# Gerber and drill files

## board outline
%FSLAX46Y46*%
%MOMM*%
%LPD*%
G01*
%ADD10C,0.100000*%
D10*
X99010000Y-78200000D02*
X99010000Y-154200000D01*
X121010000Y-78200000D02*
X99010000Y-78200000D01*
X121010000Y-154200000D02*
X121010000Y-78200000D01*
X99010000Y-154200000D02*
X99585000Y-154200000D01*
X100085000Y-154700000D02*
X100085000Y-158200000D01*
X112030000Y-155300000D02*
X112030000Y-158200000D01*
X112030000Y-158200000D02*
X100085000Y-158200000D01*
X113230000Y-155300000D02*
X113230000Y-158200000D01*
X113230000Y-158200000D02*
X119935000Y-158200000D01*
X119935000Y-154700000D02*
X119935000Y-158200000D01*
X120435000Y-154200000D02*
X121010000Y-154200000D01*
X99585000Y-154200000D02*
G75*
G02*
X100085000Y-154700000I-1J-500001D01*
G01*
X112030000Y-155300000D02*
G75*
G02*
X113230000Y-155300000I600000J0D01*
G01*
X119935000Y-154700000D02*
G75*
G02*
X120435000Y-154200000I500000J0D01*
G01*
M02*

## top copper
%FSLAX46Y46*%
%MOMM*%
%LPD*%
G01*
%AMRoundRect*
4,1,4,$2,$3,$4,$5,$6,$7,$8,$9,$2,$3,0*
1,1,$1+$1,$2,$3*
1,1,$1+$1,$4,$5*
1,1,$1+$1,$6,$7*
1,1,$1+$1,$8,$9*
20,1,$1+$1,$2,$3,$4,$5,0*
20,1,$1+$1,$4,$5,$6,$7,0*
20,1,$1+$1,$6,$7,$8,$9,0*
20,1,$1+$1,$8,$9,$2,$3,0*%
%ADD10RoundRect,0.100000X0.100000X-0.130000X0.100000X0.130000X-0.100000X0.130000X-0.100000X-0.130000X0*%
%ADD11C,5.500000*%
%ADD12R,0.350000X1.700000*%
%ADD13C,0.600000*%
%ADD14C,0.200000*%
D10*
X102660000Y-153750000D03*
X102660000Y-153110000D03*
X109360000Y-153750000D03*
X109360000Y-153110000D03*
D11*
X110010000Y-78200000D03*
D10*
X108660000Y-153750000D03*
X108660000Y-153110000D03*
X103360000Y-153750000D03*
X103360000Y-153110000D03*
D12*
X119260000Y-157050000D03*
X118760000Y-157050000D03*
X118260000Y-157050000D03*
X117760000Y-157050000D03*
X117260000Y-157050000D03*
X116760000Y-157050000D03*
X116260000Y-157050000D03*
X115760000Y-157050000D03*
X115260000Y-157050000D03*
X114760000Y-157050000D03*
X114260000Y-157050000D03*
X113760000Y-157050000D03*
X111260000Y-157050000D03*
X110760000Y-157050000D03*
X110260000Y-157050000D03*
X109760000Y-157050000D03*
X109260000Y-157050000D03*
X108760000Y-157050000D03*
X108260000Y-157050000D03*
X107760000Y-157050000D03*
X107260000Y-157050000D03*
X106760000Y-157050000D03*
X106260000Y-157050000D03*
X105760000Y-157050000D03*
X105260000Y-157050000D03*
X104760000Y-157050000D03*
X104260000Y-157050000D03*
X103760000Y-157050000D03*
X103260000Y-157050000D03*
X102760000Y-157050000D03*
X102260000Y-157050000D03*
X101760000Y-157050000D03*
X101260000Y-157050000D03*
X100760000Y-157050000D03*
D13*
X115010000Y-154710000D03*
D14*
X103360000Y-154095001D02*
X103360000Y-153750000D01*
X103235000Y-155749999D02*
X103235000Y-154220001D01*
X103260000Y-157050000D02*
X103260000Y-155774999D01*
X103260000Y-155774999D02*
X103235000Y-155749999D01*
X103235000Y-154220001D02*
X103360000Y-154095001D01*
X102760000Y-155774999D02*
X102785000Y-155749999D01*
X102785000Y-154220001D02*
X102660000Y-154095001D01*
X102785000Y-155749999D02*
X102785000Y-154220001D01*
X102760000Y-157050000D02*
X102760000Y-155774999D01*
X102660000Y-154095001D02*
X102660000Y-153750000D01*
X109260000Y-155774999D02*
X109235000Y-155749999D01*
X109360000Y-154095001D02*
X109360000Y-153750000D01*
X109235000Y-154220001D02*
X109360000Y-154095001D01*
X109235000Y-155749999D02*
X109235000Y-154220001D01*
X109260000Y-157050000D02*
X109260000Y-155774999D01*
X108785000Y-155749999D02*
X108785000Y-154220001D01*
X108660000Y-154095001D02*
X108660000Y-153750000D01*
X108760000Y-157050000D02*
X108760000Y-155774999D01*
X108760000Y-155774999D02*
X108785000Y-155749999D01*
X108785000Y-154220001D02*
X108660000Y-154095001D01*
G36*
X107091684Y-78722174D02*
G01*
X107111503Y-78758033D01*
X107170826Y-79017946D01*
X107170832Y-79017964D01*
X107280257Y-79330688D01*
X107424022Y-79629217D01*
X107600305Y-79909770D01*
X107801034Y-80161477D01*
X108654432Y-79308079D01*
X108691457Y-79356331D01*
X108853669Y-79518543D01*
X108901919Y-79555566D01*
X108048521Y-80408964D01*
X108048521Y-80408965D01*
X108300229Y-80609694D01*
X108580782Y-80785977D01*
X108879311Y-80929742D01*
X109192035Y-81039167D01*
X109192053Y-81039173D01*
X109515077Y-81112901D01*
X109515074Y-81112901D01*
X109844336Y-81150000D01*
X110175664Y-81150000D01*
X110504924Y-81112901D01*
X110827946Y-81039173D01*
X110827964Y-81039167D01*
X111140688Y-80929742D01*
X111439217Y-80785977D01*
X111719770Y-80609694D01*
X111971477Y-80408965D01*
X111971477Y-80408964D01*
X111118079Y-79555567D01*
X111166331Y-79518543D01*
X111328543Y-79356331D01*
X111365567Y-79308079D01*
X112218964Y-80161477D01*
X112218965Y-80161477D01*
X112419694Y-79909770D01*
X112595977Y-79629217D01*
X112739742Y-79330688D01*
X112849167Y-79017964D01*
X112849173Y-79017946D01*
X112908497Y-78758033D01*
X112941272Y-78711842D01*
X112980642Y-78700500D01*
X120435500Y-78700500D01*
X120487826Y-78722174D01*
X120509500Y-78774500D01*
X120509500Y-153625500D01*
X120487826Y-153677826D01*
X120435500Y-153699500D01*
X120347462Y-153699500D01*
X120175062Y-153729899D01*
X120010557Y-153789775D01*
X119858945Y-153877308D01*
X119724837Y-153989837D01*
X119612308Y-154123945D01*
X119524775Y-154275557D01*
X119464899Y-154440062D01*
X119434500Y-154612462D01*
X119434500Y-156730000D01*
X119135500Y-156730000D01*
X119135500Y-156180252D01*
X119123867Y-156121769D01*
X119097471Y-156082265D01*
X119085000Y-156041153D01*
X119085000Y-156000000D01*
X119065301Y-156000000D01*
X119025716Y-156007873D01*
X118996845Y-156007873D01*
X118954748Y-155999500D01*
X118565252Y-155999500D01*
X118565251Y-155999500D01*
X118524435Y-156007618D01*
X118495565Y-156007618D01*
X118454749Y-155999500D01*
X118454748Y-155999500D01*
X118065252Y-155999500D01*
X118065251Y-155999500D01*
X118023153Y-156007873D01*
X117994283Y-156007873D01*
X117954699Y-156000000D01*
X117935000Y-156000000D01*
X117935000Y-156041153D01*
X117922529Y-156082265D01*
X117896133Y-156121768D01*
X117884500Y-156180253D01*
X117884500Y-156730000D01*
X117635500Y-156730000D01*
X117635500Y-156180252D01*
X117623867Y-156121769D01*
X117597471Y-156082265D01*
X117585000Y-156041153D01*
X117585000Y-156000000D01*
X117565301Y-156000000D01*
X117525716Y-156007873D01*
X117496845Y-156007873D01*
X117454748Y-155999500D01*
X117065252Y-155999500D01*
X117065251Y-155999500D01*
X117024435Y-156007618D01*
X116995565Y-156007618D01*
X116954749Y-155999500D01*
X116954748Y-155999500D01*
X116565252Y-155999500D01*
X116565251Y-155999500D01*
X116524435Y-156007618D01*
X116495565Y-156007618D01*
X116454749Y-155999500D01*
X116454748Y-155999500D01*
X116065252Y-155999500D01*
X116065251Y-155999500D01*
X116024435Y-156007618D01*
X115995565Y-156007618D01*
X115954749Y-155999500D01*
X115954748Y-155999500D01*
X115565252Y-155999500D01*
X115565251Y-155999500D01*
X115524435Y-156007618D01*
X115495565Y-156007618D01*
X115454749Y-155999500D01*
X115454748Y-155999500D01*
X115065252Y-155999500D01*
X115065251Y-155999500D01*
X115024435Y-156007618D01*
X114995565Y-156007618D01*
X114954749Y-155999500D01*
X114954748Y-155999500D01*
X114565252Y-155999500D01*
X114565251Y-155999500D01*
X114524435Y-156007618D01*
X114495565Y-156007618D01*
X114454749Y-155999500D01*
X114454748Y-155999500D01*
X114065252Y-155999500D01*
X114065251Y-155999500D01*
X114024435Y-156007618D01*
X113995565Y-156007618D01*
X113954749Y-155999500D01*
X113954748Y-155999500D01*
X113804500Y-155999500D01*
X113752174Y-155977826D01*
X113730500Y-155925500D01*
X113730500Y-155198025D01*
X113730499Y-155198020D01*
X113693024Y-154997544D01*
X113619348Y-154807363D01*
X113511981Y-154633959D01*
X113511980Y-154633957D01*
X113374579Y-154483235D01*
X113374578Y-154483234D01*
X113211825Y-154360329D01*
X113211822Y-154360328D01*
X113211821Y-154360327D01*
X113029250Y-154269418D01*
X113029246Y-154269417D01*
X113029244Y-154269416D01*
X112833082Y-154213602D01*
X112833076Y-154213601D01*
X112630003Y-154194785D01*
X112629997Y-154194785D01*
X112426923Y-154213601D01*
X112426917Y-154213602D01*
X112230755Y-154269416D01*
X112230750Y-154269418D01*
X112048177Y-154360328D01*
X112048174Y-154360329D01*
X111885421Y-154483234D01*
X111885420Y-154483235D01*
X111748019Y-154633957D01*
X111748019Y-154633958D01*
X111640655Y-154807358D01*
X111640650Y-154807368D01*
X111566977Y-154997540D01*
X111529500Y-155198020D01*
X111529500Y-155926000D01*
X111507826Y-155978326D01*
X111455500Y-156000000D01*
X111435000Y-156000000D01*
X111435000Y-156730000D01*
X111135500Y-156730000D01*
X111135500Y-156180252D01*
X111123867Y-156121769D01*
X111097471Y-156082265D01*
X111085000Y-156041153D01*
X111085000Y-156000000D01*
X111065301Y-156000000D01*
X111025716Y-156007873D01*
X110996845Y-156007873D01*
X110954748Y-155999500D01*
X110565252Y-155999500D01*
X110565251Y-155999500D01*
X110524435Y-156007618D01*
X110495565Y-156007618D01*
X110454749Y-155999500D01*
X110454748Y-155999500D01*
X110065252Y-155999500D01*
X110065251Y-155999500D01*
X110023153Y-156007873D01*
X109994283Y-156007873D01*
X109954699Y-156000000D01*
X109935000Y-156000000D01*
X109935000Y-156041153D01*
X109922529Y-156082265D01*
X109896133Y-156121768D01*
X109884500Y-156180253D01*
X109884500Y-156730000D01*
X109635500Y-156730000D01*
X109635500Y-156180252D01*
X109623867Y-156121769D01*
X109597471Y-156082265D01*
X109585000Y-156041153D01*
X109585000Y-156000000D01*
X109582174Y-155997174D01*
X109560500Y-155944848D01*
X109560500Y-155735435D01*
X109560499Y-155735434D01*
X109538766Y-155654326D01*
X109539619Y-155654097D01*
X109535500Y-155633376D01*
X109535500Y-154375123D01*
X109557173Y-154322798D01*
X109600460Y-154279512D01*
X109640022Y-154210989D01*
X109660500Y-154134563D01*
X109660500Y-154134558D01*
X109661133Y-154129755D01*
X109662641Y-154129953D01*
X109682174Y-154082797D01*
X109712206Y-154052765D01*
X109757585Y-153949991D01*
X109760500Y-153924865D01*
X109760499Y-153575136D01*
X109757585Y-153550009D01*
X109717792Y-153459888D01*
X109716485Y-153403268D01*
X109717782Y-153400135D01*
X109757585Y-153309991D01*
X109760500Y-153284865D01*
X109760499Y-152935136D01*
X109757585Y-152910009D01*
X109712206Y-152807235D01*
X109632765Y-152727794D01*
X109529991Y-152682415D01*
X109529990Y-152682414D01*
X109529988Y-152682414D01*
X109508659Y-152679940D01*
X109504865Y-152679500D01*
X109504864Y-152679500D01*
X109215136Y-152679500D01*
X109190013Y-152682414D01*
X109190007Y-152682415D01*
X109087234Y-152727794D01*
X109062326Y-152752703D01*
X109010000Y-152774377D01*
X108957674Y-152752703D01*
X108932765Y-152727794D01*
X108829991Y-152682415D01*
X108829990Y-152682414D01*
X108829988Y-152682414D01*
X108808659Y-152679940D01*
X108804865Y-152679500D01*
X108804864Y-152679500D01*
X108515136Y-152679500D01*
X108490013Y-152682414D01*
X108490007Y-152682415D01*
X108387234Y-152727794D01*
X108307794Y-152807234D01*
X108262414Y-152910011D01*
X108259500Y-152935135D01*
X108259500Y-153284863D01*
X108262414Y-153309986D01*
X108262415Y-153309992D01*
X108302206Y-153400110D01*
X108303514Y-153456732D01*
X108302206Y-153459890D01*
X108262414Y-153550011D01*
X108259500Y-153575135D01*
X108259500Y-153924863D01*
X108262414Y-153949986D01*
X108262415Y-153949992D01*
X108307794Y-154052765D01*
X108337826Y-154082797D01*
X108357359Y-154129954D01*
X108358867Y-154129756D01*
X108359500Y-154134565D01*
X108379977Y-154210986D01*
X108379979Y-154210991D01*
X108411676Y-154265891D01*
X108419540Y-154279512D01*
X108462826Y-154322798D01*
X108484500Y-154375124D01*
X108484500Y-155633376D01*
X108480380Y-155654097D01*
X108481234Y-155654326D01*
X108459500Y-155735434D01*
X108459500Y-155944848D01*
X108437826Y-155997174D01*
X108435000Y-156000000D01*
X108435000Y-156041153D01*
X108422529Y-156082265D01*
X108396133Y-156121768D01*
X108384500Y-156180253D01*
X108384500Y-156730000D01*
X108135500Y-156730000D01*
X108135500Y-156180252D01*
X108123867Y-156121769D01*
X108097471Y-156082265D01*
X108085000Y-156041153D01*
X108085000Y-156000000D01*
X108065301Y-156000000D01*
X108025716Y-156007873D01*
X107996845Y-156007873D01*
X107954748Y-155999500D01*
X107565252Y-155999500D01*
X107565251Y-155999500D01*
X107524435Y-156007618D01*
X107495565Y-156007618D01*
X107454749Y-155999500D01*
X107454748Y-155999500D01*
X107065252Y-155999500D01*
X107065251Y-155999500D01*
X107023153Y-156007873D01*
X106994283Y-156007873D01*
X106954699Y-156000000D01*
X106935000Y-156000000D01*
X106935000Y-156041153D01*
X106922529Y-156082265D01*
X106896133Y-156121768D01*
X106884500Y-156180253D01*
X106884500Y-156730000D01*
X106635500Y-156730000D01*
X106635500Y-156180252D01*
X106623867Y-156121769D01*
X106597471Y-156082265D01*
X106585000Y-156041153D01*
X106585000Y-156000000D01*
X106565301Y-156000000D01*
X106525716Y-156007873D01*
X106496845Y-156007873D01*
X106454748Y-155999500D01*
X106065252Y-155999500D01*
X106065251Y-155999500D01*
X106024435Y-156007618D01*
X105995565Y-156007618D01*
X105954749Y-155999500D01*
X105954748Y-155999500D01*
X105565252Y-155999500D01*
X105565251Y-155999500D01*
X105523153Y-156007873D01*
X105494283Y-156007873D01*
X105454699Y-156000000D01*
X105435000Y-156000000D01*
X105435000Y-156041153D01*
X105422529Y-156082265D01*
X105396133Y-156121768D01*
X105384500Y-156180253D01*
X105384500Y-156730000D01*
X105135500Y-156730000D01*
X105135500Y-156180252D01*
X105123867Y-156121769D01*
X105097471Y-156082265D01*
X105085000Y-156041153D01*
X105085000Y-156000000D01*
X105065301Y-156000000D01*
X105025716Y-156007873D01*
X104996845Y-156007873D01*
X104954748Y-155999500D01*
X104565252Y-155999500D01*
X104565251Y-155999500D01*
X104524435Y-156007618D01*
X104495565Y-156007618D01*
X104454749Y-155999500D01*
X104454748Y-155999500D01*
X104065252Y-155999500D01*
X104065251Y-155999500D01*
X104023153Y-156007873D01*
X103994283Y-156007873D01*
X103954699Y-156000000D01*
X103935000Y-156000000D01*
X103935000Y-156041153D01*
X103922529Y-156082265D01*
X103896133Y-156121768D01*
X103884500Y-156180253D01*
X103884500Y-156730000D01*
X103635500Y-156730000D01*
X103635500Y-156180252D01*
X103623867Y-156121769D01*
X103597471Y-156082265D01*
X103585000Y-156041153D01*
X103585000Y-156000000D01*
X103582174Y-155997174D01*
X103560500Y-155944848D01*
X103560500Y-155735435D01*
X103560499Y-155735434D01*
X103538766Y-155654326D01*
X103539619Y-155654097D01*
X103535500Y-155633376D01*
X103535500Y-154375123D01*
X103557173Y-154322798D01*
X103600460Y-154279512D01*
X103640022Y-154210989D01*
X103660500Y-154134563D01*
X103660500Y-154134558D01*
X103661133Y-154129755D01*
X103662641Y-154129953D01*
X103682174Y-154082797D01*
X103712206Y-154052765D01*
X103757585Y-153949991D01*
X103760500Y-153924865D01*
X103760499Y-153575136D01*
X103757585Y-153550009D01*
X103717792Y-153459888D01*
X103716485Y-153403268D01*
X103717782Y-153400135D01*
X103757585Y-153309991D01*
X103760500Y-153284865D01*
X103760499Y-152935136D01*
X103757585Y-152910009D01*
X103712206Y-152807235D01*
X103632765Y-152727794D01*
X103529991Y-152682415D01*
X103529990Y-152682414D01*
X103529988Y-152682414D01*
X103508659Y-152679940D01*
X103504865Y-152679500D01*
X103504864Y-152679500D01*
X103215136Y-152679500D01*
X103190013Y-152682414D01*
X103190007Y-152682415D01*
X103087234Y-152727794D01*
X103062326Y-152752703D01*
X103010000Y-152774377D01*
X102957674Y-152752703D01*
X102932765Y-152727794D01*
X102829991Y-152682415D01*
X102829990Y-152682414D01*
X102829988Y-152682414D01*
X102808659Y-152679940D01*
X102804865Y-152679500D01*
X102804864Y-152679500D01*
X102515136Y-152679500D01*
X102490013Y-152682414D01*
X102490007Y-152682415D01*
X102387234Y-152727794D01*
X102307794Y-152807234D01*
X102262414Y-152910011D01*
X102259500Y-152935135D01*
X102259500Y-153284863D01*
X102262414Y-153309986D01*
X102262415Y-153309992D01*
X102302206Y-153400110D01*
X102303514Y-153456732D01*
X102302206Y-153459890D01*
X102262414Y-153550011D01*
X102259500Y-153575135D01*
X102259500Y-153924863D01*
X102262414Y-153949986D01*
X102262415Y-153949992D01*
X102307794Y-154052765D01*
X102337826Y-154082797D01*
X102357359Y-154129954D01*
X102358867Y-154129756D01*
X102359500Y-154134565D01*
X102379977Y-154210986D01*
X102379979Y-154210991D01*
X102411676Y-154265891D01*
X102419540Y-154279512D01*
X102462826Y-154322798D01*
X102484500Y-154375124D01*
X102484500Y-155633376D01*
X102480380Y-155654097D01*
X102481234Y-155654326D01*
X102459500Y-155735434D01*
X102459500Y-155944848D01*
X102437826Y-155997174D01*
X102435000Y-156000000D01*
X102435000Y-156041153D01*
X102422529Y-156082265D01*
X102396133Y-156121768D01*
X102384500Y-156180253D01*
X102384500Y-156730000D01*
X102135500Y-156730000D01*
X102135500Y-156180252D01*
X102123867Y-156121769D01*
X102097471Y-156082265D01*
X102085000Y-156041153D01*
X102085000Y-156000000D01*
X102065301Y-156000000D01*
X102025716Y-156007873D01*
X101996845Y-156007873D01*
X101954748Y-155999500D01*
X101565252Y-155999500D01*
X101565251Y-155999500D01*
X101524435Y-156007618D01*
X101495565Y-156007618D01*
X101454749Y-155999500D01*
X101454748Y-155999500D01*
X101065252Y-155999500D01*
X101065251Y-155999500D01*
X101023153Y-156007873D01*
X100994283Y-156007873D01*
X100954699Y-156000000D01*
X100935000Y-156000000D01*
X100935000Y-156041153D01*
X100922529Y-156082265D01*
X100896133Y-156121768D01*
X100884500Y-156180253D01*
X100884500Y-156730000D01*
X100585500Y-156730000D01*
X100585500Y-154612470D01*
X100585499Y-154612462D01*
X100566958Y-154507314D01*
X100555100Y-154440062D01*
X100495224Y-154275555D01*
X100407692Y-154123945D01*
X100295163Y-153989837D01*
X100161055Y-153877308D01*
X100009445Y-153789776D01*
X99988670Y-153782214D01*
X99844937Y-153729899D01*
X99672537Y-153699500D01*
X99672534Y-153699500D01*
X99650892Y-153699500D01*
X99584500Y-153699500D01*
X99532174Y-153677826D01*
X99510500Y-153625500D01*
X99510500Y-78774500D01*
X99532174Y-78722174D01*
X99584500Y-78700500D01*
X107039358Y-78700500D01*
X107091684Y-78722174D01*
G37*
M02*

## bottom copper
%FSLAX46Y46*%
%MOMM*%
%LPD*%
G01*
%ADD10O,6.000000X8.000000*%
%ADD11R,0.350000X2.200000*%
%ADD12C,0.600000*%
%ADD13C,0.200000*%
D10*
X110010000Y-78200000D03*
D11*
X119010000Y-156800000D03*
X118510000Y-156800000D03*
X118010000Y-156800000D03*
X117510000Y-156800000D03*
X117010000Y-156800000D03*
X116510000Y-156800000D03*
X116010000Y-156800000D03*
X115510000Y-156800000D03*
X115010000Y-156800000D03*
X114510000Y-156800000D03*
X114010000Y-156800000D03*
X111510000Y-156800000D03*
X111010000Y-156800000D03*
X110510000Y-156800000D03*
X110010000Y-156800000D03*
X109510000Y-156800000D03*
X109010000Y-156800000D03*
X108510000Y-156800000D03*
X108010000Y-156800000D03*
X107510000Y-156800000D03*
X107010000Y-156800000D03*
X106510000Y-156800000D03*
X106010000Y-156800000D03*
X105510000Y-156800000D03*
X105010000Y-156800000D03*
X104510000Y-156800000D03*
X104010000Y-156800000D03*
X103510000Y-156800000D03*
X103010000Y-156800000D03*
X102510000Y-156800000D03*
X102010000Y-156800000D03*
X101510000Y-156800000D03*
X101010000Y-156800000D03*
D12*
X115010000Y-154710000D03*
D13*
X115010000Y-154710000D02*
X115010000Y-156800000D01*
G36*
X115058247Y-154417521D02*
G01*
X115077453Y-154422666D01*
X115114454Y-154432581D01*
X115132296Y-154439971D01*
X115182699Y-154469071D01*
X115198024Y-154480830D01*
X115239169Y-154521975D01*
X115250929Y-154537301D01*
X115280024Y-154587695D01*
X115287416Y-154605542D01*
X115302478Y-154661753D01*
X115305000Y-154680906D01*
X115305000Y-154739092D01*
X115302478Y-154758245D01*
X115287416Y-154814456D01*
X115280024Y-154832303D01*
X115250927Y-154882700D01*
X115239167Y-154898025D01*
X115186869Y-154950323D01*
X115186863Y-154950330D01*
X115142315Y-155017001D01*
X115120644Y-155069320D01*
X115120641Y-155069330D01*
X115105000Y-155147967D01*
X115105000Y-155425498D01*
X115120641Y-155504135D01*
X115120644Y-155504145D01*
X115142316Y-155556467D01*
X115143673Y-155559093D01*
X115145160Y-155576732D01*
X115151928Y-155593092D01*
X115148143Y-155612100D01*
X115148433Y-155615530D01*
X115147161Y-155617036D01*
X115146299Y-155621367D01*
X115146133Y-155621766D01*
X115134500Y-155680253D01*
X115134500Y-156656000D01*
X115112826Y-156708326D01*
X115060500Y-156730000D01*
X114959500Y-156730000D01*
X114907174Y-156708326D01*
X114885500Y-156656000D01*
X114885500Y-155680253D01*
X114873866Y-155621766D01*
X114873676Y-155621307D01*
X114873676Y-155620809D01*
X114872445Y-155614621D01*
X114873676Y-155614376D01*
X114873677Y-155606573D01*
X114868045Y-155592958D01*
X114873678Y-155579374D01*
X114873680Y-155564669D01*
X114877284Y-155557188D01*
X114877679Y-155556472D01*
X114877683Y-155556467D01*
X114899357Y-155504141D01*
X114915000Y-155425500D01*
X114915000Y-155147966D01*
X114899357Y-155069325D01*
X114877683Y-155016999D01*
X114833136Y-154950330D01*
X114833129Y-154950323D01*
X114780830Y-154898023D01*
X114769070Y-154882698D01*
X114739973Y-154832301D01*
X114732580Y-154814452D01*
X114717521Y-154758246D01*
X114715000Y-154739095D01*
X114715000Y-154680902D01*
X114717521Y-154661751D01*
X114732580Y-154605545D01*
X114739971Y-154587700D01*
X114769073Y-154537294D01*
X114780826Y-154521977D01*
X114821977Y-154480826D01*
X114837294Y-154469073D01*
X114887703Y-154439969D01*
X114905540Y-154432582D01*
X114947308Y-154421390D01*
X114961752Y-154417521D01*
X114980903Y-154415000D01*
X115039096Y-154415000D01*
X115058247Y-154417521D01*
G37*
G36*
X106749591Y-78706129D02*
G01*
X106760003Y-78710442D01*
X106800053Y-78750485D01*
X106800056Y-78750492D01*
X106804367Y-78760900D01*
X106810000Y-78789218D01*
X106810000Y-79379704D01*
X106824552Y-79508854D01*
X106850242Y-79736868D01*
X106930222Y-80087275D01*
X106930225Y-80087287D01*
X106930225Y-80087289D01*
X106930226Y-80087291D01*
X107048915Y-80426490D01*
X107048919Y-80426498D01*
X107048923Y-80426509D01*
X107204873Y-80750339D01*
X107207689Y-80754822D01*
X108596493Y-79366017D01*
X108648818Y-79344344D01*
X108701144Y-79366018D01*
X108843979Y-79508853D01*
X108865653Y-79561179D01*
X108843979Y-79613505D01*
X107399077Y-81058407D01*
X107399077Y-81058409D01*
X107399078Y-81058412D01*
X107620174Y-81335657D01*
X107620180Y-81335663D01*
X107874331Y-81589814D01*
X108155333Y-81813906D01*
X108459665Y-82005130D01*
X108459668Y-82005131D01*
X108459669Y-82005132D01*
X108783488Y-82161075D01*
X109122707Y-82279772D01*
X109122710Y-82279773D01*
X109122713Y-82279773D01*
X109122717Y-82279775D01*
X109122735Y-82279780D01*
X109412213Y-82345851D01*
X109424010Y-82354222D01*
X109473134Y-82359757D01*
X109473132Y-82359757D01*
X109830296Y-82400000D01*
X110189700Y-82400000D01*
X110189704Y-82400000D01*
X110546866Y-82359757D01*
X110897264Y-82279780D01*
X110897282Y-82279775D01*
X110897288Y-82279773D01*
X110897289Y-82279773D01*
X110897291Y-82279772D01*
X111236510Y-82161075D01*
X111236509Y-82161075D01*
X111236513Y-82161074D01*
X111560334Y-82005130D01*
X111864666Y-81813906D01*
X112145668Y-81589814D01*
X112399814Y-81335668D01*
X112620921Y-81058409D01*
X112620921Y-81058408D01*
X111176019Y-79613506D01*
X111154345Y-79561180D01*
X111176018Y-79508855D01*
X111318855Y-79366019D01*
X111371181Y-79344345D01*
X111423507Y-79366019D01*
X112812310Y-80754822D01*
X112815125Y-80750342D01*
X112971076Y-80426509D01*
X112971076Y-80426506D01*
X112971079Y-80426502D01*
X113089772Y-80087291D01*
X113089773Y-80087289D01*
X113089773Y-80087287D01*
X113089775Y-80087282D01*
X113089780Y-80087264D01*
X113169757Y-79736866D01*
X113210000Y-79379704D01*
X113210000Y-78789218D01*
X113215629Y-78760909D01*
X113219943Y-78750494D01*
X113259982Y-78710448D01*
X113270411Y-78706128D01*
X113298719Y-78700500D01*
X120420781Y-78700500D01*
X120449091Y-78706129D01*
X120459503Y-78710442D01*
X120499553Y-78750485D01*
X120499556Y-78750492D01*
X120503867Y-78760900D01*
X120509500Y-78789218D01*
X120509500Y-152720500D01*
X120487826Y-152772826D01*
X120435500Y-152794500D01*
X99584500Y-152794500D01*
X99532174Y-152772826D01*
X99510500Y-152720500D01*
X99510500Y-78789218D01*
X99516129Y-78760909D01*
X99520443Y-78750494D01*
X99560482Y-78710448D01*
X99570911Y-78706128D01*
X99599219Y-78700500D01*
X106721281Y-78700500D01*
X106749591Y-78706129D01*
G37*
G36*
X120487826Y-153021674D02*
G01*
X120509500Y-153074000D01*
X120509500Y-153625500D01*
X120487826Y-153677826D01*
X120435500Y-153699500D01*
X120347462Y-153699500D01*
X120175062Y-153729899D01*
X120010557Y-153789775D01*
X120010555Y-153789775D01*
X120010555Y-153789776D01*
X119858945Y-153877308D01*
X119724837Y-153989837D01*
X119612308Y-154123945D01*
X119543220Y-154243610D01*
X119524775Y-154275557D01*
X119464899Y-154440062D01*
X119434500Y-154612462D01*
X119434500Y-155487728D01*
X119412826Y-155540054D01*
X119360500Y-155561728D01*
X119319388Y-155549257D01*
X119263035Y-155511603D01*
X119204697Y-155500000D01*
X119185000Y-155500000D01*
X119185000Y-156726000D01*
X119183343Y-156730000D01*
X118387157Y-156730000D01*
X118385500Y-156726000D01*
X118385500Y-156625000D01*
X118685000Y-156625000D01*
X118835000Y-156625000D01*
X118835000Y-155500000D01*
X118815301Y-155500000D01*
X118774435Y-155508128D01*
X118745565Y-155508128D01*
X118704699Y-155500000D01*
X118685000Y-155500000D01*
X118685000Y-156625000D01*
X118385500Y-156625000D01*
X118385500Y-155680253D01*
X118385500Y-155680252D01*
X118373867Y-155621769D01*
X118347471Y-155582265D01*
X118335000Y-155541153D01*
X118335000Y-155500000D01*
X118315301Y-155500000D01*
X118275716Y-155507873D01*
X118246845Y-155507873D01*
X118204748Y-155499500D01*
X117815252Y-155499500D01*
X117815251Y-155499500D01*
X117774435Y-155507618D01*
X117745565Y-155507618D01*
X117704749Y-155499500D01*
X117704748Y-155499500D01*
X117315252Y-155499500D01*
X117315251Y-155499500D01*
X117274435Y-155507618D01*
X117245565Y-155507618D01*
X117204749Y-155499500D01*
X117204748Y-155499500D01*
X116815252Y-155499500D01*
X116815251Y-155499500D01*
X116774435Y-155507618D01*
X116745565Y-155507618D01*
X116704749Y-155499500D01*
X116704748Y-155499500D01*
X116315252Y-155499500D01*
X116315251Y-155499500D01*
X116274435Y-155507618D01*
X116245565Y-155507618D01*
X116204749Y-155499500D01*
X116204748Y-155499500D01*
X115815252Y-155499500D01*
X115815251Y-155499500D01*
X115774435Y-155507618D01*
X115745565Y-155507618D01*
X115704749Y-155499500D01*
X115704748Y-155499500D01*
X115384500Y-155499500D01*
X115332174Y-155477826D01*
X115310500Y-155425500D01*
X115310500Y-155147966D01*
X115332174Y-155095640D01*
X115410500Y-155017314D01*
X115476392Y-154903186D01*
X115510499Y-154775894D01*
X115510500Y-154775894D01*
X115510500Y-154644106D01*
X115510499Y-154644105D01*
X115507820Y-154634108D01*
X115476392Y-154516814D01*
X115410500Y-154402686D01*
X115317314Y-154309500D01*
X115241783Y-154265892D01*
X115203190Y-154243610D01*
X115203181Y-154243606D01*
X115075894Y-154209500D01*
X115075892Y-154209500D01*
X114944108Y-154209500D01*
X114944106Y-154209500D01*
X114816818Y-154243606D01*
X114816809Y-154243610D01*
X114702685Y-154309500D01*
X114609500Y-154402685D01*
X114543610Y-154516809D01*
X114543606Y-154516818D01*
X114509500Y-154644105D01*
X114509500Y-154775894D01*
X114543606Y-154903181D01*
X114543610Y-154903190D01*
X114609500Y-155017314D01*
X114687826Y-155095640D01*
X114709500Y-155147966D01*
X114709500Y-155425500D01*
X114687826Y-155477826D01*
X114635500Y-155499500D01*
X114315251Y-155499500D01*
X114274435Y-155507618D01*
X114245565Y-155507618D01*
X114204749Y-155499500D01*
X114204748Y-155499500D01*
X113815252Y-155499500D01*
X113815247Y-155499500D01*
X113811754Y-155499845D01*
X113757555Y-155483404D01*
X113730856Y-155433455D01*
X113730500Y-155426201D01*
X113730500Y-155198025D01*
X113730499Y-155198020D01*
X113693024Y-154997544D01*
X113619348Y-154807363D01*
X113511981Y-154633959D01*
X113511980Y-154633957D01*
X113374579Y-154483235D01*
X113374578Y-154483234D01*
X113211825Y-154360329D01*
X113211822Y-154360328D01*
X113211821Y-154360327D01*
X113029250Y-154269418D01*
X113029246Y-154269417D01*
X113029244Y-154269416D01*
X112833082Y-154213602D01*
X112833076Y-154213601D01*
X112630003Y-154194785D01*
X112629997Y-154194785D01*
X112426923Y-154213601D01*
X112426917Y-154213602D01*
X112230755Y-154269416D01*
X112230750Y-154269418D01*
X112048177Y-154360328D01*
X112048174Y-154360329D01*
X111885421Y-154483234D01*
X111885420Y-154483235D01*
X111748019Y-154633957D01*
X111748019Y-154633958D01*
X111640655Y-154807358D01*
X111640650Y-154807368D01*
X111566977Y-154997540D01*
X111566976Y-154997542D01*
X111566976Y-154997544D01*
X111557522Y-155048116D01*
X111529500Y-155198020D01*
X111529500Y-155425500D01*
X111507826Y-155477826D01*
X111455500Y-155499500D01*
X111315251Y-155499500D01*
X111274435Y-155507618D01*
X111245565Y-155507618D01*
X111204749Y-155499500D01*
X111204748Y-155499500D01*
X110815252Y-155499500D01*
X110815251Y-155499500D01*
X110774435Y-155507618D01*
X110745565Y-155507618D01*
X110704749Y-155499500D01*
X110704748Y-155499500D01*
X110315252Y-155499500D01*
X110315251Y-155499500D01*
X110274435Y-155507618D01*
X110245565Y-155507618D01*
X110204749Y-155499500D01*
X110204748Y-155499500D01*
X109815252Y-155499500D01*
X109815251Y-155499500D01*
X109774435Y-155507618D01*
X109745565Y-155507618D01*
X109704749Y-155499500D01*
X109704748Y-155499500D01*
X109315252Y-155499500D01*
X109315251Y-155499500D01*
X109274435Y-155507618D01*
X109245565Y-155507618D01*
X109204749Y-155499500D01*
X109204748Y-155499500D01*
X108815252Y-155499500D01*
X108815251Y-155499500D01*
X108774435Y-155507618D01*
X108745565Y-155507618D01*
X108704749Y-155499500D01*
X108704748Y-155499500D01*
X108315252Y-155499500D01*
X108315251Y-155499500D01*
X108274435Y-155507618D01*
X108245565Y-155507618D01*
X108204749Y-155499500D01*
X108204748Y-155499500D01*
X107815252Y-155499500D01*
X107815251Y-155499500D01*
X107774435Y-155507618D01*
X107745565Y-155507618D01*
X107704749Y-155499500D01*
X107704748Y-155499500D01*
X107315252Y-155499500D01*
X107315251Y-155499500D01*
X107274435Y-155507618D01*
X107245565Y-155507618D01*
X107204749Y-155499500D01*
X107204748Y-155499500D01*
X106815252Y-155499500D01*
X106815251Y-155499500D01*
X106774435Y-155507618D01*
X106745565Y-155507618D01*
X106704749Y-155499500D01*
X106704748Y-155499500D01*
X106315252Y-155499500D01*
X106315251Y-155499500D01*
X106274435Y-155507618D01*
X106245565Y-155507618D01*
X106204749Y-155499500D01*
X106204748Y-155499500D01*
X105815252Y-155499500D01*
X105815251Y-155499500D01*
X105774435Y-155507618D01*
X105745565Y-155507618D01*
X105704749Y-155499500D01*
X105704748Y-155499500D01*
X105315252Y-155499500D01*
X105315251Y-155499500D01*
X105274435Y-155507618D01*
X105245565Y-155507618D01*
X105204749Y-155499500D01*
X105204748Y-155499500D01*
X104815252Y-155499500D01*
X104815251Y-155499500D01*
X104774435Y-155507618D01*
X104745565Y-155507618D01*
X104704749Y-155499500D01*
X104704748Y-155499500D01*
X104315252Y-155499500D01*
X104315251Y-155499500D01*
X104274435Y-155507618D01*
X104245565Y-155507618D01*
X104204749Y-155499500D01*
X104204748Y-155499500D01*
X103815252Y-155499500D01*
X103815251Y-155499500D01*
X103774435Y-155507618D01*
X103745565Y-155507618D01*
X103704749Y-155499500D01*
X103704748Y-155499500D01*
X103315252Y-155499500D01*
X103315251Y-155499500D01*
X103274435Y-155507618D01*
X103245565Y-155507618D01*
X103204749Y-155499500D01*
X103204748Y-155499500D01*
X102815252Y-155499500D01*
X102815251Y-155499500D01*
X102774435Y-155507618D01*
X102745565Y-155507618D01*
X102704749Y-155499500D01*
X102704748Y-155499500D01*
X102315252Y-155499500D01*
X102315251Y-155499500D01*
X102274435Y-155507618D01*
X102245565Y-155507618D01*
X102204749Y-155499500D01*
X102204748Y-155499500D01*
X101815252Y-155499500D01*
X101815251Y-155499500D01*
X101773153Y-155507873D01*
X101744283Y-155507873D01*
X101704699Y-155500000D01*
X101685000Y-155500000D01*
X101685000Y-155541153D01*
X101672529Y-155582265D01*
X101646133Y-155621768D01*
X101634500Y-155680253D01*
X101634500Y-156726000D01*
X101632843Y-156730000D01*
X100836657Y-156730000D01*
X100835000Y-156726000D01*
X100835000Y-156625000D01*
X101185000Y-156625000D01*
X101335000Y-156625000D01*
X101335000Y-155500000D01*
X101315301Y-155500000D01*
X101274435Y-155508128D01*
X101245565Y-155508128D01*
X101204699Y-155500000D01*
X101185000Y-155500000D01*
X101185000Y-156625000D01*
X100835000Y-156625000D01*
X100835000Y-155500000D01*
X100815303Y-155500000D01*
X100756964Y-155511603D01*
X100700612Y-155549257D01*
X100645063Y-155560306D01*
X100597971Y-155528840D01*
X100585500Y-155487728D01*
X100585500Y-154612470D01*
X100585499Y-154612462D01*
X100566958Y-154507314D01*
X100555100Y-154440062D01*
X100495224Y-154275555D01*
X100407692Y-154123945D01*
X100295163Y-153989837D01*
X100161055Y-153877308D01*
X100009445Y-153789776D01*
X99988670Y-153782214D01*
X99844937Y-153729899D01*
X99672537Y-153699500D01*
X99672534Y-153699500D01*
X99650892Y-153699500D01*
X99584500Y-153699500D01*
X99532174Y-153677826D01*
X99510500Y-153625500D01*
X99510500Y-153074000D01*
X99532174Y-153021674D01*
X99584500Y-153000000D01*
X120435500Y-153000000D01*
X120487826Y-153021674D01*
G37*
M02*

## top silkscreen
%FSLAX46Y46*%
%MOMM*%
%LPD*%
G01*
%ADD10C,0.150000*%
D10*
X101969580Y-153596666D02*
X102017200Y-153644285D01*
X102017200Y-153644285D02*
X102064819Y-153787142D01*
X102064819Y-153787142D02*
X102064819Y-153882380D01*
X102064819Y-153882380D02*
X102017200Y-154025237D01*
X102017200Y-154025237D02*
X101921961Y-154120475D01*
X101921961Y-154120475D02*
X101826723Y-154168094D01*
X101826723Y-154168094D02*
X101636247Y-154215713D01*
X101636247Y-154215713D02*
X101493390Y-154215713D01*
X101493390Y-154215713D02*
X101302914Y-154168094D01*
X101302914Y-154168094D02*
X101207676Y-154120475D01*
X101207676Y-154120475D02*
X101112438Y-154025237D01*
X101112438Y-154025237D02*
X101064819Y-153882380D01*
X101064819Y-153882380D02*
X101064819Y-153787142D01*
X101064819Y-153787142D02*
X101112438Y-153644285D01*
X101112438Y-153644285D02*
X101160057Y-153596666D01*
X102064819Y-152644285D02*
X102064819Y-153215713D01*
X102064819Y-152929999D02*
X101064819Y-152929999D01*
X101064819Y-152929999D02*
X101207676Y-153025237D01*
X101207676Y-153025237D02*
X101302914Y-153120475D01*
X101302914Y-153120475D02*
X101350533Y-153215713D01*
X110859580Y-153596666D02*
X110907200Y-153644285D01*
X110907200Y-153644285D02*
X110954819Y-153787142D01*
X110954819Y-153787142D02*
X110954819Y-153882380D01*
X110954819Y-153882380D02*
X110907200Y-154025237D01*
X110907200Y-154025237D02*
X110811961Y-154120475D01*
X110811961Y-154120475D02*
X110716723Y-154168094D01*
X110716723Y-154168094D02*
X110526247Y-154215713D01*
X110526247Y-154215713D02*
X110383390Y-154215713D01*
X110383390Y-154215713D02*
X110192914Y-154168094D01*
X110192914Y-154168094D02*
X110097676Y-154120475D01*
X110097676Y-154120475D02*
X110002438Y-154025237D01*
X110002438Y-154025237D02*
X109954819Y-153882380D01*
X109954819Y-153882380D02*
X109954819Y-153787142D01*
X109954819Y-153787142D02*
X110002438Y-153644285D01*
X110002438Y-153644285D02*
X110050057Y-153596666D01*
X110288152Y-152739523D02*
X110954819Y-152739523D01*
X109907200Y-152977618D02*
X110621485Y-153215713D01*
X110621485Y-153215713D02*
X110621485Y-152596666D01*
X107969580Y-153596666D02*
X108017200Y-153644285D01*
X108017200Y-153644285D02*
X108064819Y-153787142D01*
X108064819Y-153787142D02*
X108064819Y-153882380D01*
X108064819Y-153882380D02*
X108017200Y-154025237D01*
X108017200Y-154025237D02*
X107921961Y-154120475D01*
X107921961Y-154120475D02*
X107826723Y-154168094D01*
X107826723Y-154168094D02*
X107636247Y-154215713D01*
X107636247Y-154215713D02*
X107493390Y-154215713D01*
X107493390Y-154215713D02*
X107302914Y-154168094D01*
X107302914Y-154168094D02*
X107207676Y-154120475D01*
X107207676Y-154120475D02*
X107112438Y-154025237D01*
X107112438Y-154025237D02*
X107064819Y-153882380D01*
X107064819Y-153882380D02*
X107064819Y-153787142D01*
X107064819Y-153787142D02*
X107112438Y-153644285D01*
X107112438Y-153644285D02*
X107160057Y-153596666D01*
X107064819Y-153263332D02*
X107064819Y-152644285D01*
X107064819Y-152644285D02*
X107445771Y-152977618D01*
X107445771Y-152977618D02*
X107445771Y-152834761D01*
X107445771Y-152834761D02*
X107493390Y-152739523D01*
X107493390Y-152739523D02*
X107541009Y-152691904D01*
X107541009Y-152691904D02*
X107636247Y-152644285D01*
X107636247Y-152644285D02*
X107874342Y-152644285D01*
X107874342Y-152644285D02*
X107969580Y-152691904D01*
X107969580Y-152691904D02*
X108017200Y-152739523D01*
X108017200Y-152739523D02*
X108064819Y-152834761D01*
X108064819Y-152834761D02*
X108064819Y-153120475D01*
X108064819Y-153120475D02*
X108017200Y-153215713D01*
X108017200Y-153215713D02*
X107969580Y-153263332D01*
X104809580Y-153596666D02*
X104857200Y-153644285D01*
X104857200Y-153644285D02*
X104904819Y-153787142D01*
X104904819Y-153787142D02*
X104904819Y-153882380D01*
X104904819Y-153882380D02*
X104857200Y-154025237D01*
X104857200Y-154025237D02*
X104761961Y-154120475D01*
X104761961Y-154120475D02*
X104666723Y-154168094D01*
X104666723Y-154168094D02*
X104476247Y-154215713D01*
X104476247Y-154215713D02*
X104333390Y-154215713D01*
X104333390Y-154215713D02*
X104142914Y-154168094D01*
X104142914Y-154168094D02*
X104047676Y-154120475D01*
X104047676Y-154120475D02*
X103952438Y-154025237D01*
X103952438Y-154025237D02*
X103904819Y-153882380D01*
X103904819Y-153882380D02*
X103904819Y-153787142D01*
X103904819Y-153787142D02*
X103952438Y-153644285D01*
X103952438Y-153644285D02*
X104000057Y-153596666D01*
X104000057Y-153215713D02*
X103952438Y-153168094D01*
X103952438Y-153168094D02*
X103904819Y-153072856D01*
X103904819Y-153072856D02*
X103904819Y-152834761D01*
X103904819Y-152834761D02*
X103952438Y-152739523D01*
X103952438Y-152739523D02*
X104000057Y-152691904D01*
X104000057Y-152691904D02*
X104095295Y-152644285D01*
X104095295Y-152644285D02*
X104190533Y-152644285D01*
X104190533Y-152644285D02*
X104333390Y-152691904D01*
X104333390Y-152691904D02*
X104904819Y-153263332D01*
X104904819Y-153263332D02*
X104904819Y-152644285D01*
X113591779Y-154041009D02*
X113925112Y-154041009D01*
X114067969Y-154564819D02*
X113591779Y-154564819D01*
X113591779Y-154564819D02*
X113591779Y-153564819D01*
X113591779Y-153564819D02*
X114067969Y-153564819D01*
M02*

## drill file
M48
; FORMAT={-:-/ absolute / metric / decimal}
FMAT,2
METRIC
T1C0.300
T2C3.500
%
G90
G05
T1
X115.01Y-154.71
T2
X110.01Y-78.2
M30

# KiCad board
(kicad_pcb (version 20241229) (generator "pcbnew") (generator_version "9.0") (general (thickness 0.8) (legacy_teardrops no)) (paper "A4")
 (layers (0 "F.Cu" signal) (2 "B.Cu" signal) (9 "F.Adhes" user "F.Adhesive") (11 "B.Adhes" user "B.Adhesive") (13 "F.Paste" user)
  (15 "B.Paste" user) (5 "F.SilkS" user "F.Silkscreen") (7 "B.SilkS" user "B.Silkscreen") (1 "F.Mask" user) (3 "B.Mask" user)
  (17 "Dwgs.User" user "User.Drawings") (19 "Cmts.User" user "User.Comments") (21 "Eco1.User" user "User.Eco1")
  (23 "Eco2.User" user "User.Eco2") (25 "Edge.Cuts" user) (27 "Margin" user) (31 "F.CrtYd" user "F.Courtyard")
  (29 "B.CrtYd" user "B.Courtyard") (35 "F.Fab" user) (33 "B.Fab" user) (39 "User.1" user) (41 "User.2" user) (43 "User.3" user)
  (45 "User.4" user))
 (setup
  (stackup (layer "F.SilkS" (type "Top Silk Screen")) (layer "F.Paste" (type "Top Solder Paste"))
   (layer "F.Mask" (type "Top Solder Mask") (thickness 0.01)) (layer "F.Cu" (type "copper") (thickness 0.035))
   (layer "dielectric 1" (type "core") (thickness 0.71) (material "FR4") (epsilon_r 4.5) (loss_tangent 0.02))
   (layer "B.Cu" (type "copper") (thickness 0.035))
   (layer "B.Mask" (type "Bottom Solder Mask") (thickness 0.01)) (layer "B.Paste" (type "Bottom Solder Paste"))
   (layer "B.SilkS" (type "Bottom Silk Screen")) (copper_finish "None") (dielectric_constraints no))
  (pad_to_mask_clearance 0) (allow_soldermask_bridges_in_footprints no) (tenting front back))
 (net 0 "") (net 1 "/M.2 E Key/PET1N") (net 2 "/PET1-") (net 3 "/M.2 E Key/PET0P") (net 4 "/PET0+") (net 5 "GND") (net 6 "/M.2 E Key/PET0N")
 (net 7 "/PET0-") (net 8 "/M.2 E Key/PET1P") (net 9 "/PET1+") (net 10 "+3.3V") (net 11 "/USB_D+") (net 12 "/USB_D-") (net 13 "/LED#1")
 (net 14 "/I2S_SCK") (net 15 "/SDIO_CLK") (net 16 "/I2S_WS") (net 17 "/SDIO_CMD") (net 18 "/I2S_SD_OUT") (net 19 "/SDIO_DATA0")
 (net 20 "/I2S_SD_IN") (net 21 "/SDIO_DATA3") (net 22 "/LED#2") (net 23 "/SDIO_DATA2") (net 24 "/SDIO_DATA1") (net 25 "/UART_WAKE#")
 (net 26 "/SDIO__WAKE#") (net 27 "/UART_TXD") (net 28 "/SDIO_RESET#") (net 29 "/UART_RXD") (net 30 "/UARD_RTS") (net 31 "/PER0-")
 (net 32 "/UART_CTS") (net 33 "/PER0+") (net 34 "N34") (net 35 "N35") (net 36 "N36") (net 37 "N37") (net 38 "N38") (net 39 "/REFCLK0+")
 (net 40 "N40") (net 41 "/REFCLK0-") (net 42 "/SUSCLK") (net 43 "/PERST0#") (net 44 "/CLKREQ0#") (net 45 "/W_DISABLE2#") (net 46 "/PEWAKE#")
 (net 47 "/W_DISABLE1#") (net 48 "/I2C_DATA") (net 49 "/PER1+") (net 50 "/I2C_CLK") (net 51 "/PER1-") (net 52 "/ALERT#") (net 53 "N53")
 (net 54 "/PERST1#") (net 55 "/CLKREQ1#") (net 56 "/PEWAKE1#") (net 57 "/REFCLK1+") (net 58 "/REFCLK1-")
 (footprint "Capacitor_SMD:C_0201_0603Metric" (layer "F.Cu") (at 102.66 153.43 90)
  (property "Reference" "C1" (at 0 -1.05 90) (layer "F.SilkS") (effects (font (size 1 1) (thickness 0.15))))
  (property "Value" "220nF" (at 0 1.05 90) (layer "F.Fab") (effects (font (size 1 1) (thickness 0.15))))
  (pad "" smd roundrect (at -0.345 0 90) (size 0.318 0.36) (layers "F.Paste") (roundrect_rratio 0.25))
  (pad "" smd roundrect (at 0.345 0 90) (size 0.318 0.36) (layers "F.Paste") (roundrect_rratio 0.25))
  (pad "1" smd roundrect (at -0.32 0 90) (size 0.46 0.4) (layers "F.Cu" "F.Mask") (roundrect_rratio 0.25) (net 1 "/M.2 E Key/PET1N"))
  (pad "2" smd roundrect (at 0.32 0 90) (size 0.46 0.4) (layers "F.Cu" "F.Mask") (roundrect_rratio 0.25) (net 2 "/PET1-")))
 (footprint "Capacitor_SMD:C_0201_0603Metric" (layer "F.Cu") (at 109.36 153.43 90)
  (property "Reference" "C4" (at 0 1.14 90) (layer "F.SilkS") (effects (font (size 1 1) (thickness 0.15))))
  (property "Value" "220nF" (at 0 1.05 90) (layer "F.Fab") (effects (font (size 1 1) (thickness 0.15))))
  (pad "" smd roundrect (at -0.345 0 90) (size 0.318 0.36) (layers "F.Paste") (roundrect_rratio 0.25))
  (pad "" smd roundrect (at 0.345 0 90) (size 0.318 0.36) (layers "F.Paste") (roundrect_rratio 0.25))
  (pad "1" smd roundrect (at -0.32 0 90) (size 0.46 0.4) (layers "F.Cu" "F.Mask") (roundrect_rratio 0.25) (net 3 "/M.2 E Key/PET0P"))
  (pad "2" smd roundrect (at 0.32 0 90) (size 0.46 0.4) (layers "F.Cu" "F.Mask") (roundrect_rratio 0.25) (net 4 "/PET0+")))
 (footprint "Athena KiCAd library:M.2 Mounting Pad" (layer "F.Cu") (at 110.01 78.2)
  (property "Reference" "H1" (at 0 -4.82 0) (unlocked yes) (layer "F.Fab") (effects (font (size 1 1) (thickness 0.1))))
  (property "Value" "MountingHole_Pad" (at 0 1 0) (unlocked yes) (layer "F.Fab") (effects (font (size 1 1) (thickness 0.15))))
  (pad "1" thru_hole circle (at 0 0) (size 5.5 5.5) (drill 3.5) (layers "*.Cu" "*.Mask") (remove_unused_layers no) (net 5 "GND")
   (padstack (mode front_inner_back)
    (layer "Inner" (shape circle) (size 5.5 5.5) (zone_connect -1))
    (layer "B.Cu" (shape oval) (size 6 8) (thermal_bridge_angle 45) (zone_connect -1)))))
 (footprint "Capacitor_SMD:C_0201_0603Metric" (layer "F.Cu") (at 108.66 153.43 90)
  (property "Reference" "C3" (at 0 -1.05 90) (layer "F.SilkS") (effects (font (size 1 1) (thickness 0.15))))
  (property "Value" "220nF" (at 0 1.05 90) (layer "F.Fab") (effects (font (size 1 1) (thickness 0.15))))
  (pad "" smd roundrect (at -0.345 0 90) (size 0.318 0.36) (layers "F.Paste") (roundrect_rratio 0.25))
  (pad "" smd roundrect (at 0.345 0 90) (size 0.318 0.36) (layers "F.Paste") (roundrect_rratio 0.25))
  (pad "1" smd roundrect (at -0.32 0 90) (size 0.46 0.4) (layers "F.Cu" "F.Mask") (roundrect_rratio 0.25) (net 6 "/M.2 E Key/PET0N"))
  (pad "2" smd roundrect (at 0.32 0 90) (size 0.46 0.4) (layers "F.Cu" "F.Mask") (roundrect_rratio 0.25) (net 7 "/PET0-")))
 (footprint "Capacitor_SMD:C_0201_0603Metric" (layer "F.Cu") (at 103.36 153.43 90)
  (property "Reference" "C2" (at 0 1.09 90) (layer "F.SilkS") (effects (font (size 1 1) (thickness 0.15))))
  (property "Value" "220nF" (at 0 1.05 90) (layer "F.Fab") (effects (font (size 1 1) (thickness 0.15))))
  (pad "" smd roundrect (at -0.345 0 90) (size 0.318 0.36) (layers "F.Paste") (roundrect_rratio 0.25))
  (pad "" smd roundrect (at 0.345 0 90) (size 0.318 0.36) (layers "F.Paste") (roundrect_rratio 0.25))
  (pad "1" smd roundrect (at -0.32 0 90) (size 0.46 0.4) (layers "F.Cu" "F.Mask") (roundrect_rratio 0.25) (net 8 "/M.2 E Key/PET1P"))
  (pad "2" smd roundrect (at 0.32 0 90) (size 0.46 0.4) (layers "F.Cu" "F.Mask") (roundrect_rratio 0.25) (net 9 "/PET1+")))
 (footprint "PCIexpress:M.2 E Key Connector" (layer "F.Cu") (at 110.01 157.09)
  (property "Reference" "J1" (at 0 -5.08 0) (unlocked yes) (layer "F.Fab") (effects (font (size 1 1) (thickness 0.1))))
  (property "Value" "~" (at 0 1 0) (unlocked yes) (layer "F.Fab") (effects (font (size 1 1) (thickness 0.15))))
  (fp_line (start -11 -2.89) (end -10.425 -2.89) (stroke (width 0.1) (type default)) (layer "Edge.Cuts") (net 8))
  (fp_line (start -9.925 -2.39) (end -9.925 1.11) (stroke (width 0.1) (type default)) (layer "Edge.Cuts") (net 8))
  (fp_line (start 2.02 -1.79) (end 2.02 1.11) (stroke (width 0.1) (type default)) (layer "Edge.Cuts") (net 8))
  (fp_line (start 2.02 1.11) (end -9.925 1.11) (stroke (width 0.1) (type default)) (layer "Edge.Cuts") (net 8))
  (fp_line (start 3.22 -1.79) (end 3.22 1.11) (stroke (width 0.1) (type default)) (layer "Edge.Cuts") (net 8))
  (fp_line (start 3.22 1.11) (end 9.925 1.11) (stroke (width 0.1) (type default)) (layer "Edge.Cuts") (net 8))
  (fp_line (start 9.925 -2.39) (end 9.925 1.11) (stroke (width 0.1) (type default)) (layer "Edge.Cuts") (net 8))
  (fp_line (start 10.425 -2.89) (end 11 -2.89) (stroke (width 0.1) (type default)) (layer "Edge.Cuts") (net 8))
  (fp_arc (start -10.425 -2.89) (mid -10.071447 -2.743553) (end -9.925 -2.39) (stroke (width 0.1) (type default)) (layer "Edge.Cuts")
   (net 8))
  (fp_arc (start 2.02 -1.79) (mid 2.62 -2.39) (end 3.22 -1.79) (stroke (width 0.1) (type default)) (layer "Edge.Cuts") (net 8))
  (fp_arc (start 9.925 -2.39) (mid 10.071447 -2.743553) (end 10.425 -2.89) (stroke (width 0.1) (type default)) (layer "Edge.Cuts") (net 8))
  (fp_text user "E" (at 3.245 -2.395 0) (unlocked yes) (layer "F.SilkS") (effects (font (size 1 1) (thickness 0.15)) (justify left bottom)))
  (pad "1" smd rect (at 9.25 -0.04 180) (size 0.35 1.7) (layers "F.Cu") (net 5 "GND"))
  (pad "2" smd rect (at 9 -0.29 180) (size 0.35 2.2) (layers "B.Cu") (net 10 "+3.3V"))
  (pad "3" smd rect (at 8.75 -0.04 180) (size 0.35 1.7) (layers "F.Cu") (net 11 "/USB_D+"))
  (pad "4" smd rect (at 8.5 -0.29 180) (size 0.35 2.2) (layers "B.Cu") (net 10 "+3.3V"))
  (pad "5" smd rect (at 8.25 -0.04 180) (size 0.35 1.7) (layers "F.Cu") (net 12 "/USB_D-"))
  (pad "6" smd rect (at 8 -0.29 180) (size 0.35 2.2) (layers "B.Cu") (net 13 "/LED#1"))
  (pad "7" smd rect (at 7.75 -0.04 180) (size 0.35 1.7) (layers "F.Cu") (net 5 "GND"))
  (pad "8" smd rect (at 7.5 -0.29 180) (size 0.35 2.2) (layers "B.Cu") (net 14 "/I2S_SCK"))
  (pad "9" smd rect (at 7.25 -0.04 180) (size 0.35 1.7) (layers "F.Cu") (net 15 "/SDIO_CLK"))
  (pad "10" smd rect (at 7 -0.29 180) (size 0.35 2.2) (layers "B.Cu") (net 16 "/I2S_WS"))
  (pad "11" smd rect (at 6.75 -0.04 180) (size 0.35 1.7) (layers "F.Cu") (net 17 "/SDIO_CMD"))
  (pad "12" smd rect (at 6.5 -0.29 180) (size 0.35 2.2) (layers "B.Cu") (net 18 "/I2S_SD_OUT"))
  (pad "13" smd rect (at 6.25 -0.04 180) (size 0.35 1.7) (layers "F.Cu") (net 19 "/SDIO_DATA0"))
  (pad "14" smd rect (at 6 -0.29 180) (size 0.35 2.2) (layers "B.Cu") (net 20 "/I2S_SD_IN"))
  (pad "15" smd rect (at 5.75 -0.04 180) (size 0.35 1.7) (layers "F.Cu") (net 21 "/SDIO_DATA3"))
  (pad "16" smd rect (at 5.5 -0.29 180) (size 0.35 2.2) (layers "B.Cu") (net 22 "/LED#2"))
  (pad "17" smd rect (at 5.25 -0.04 180) (size 0.35 1.7) (layers "F.Cu") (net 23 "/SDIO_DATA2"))
  (pad "18" smd rect (at 5 -0.29 180) (size 0.35 2.2) (layers "B.Cu") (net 5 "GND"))
  (pad "19" smd rect (at 4.75 -0.04 180) (size 0.35 1.7) (layers "F.Cu") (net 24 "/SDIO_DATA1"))
  (pad "20" smd rect (at 4.5 -0.29 180) (size 0.35 2.2) (layers "B.Cu") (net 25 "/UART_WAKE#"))
  (pad "21" smd rect (at 4.25 -0.04 180) (size 0.35 1.7) (layers "F.Cu") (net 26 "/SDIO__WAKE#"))
  (pad "22" smd rect (at 4 -0.29 180) (size 0.35 2.2) (layers "B.Cu") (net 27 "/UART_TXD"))
  (pad "23" smd rect (at 3.75 -0.04 180) (size 0.35 1.7) (layers "F.Cu") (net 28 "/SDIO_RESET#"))
  (pad "32" smd rect (at 1.5 -0.29 180) (size 0.35 2.2) (layers "B.Cu") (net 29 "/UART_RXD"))
  (pad "33" smd rect (at 1.25 -0.04 180) (size 0.35 1.7) (layers "F.Cu") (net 5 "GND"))
  (pad "34" smd rect (at 1 -0.29 180) (size 0.35 2.2) (layers "B.Cu") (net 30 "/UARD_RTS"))
  (pad "35" smd rect (at 0.75 -0.04 180) (size 0.35 1.7) (layers "F.Cu") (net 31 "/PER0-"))
  (pad "36" smd rect (at 0.5 -0.29 180) (size 0.35 2.2) (layers "B.Cu") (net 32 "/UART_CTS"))
  (pad "37" smd rect (at 0.25 -0.04 180) (size 0.35 1.7) (layers "F.Cu") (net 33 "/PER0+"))
  (pad "38" smd rect (at 0 -0.29 180) (size 0.35 2.2) (layers "B.Cu") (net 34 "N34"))
  (pad "39" smd rect (at -0.25 -0.04 180) (size 0.35 1.7) (layers "F.Cu") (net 5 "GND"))
  (pad "40" smd rect (at -0.5 -0.29 180) (size 0.35 2.2) (layers "B.Cu") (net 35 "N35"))
  (pad "41" smd rect (at -0.75 -0.04 180) (size 0.35 1.7) (layers "F.Cu") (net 3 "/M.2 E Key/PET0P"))
  (pad "42" smd rect (at -1 -0.29 180) (size 0.35 2.2) (layers "B.Cu") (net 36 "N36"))
  (pad "43" smd rect (at -1.25 -0.04 180) (size 0.35 1.7) (layers "F.Cu") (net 6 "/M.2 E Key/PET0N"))
  (pad "44" smd rect (at -1.5 -0.29 180) (size 0.35 2.2) (layers "B.Cu") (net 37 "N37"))
  (pad "45" smd rect (at -1.75 -0.04 180) (size 0.35 1.7) (layers "F.Cu") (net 5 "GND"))
  (pad "46" smd rect (at -2 -0.29 180) (size 0.35 2.2) (layers "B.Cu") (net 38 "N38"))
  (pad "47" smd rect (at -2.25 -0.04 180) (size 0.35 1.7) (layers "F.Cu") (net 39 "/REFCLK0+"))
  (pad "48" smd rect (at -2.5 -0.29 180) (size 0.35 2.2) (layers "B.Cu") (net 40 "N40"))
  (pad "49" smd rect (at -2.75 -0.04 180) (size 0.35 1.7) (layers "F.Cu") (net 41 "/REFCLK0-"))
  (pad "50" smd rect (at -3 -0.29 180) (size 0.35 2.2) (layers "B.Cu") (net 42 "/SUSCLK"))
  (pad "51" smd rect (at -3.25 -0.04 180) (size 0.35 1.7) (layers "F.Cu") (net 5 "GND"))
  (pad "52" smd rect (at -3.5 -0.29 180) (size 0.35 2.2) (layers "B.Cu") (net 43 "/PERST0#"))
  (pad "53" smd rect (at -3.75 -0.04 180) (size 0.35 1.7) (layers "F.Cu") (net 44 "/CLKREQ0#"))
  (pad "54" smd rect (at -4 -0.29 180) (size 0.35 2.2) (layers "B.Cu") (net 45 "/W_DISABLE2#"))
  (pad "55" smd rect (at -4.25 -0.04 180) (size 0.35 1.7) (layers "F.Cu") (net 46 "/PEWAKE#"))
  (pad "56" smd rect (at -4.5 -0.29 180) (size 0.35 2.2) (layers "B.Cu") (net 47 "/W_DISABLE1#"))
  (pad "57" smd rect (at -4.75 -0.04 180) (size 0.35 1.7) (layers "F.Cu") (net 5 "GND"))
  (pad "58" smd rect (at -5 -0.29 180) (size 0.35 2.2) (layers "B.Cu") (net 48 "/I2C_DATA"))
  (pad "59" smd rect (at -5.25 -0.04 180) (size 0.35 1.7) (layers "F.Cu") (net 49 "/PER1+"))
  (pad "60" smd rect (at -5.5 -0.29 180) (size 0.35 2.2) (layers "B.Cu") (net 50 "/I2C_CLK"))
  (pad "61" smd rect (at -5.75 -0.04 180) (size 0.35 1.7) (layers "F.Cu") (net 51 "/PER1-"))
  (pad "62" smd rect (at -6 -0.29 180) (size 0.35 2.2) (layers "B.Cu") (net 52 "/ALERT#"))
  (pad "63" smd rect (at -6.25 -0.04 180) (size 0.35 1.7) (layers "F.Cu") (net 5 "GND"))
  (pad "64" smd rect (at -6.5 -0.29 180) (size 0.35 2.2) (layers "B.Cu") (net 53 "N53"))
  (pad "65" smd rect (at -6.75 -0.04 180) (size 0.35 1.7) (layers "F.Cu") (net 8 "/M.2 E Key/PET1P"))
  (pad "66" smd rect (at -7 -0.29 180) (size 0.35 2.2) (layers "B.Cu") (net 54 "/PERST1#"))
  (pad "67" smd rect (at -7.25 -0.04 180) (size 0.35 1.7) (layers "F.Cu") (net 1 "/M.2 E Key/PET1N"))
  (pad "68" smd rect (at -7.5 -0.29 180) (size 0.35 2.2) (layers "B.Cu") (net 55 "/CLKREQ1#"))
  (pad "69" smd rect (at -7.75 -0.04 180) (size 0.35 1.7) (layers "F.Cu") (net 5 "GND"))
  (pad "70" smd rect (at -8 -0.29 180) (size 0.35 2.2) (layers "B.Cu") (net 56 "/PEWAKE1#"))
  (pad "71" smd rect (at -8.25 -0.04 180) (size 0.35 1.7) (layers "F.Cu") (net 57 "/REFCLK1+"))
  (pad "72" smd rect (at -8.5 -0.29 180) (size 0.35 2.2) (layers "B.Cu") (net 10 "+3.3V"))
  (pad "73" smd rect (at -8.75 -0.04 180) (size 0.35 1.7) (layers "F.Cu") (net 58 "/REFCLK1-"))
  (pad "74" smd rect (at -9 -0.29 180) (size 0.35 2.2) (layers "B.Cu") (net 10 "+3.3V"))
  (pad "75" smd rect (at -9.25 -0.04 180) (size 0.35 1.7) (layers "F.Cu") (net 5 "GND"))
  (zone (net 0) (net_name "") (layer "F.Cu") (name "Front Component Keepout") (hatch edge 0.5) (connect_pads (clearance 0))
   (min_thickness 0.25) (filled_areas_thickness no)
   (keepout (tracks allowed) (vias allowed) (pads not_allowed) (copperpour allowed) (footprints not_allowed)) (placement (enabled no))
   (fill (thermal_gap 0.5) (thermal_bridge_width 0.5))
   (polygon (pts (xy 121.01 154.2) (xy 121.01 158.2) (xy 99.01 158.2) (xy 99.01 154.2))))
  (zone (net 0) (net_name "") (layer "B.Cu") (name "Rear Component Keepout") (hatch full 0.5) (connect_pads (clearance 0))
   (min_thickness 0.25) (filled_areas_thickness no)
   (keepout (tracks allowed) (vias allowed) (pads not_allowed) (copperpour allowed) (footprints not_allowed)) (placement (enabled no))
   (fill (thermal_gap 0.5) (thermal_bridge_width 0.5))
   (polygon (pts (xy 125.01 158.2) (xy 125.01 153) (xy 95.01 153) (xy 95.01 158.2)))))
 (gr_line (start 99.01 78.2) (end 99.01 154.2) (stroke (width 0.1) (type default)) (layer "Edge.Cuts"))
 (gr_line (start 121.01 78.2) (end 99.01 78.2) (stroke (width 0.1) (type default)) (layer "Edge.Cuts"))
 (gr_line (start 121.01 154.2) (end 121.01 78.2) (stroke (width 0.1) (type default)) (layer "Edge.Cuts"))
 (segment (start 103.36 154.095001) (end 103.36 153.75) (width 0.2) (layer "F.Cu") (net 8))
 (segment (start 103.235 155.749999) (end 103.235 154.220001) (width 0.2) (layer "F.Cu") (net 8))
 (segment (start 103.26 157.05) (end 103.26 155.774999) (width 0.2) (layer "F.Cu") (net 8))
 (segment (start 103.26 155.774999) (end 103.235 155.749999) (width 0.2) (layer "F.Cu") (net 8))
 (segment (start 103.235 154.220001) (end 103.36 154.095001) (width 0.2) (layer "F.Cu") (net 8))
 (segment (start 102.76 155.774999) (end 102.785 155.749999) (width 0.2) (layer "F.Cu") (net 1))
 (segment (start 102.785 154.220001) (end 102.66 154.095001) (width 0.2) (layer "F.Cu") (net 1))
 (segment (start 102.785 155.749999) (end 102.785 154.220001) (width 0.2) (layer "F.Cu") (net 1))
 (segment (start 102.76 157.05) (end 102.76 155.774999) (width 0.2) (layer "F.Cu") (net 1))
 (segment (start 102.66 154.095001) (end 102.66 153.75) (width 0.2) (layer "F.Cu") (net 1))
 (segment (start 109.26 155.774999) (end 109.235 155.749999) (width 0.2) (layer "F.Cu") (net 3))
 (segment (start 109.36 154.095001) (end 109.36 153.75) (width 0.2) (layer "F.Cu") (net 3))
 (segment (start 109.235 154.220001) (end 109.36 154.095001) (width 0.2) (layer "F.Cu") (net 3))
 (segment (start 109.235 155.749999) (end 109.235 154.220001) (width 0.2) (layer "F.Cu") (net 3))
 (segment (start 109.26 157.05) (end 109.26 155.774999) (width 0.2) (layer "F.Cu") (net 3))
 (segment (start 108.785 155.749999) (end 108.785 154.220001) (width 0.2) (layer "F.Cu") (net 6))
 (segment (start 108.66 154.095001) (end 108.66 153.75) (width 0.2) (layer "F.Cu") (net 6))
 (segment (start 108.76 157.05) (end 108.76 155.774999) (width 0.2) (layer "F.Cu") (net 6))
 (segment (start 108.76 155.774999) (end 108.785 155.749999) (width 0.2) (layer "F.Cu") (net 6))
 (segment (start 108.785 154.220001) (end 108.66 154.095001) (width 0.2) (layer "F.Cu") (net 6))
 (via (at 115.01 154.71) (size 0.6) (drill 0.3) (layers "F.Cu" "B.Cu") (free yes) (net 5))
 (segment (start 115.01 154.71) (end 115.01 156.8) (width 0.2) (layer "B.Cu") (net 5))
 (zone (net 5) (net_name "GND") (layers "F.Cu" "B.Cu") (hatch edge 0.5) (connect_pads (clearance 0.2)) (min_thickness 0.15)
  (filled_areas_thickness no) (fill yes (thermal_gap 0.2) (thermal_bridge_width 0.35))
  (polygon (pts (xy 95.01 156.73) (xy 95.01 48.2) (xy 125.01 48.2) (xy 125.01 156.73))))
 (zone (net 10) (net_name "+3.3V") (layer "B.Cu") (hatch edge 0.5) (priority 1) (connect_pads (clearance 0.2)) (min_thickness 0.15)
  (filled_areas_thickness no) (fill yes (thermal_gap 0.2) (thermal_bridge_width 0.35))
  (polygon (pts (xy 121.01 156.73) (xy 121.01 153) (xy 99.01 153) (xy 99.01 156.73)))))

